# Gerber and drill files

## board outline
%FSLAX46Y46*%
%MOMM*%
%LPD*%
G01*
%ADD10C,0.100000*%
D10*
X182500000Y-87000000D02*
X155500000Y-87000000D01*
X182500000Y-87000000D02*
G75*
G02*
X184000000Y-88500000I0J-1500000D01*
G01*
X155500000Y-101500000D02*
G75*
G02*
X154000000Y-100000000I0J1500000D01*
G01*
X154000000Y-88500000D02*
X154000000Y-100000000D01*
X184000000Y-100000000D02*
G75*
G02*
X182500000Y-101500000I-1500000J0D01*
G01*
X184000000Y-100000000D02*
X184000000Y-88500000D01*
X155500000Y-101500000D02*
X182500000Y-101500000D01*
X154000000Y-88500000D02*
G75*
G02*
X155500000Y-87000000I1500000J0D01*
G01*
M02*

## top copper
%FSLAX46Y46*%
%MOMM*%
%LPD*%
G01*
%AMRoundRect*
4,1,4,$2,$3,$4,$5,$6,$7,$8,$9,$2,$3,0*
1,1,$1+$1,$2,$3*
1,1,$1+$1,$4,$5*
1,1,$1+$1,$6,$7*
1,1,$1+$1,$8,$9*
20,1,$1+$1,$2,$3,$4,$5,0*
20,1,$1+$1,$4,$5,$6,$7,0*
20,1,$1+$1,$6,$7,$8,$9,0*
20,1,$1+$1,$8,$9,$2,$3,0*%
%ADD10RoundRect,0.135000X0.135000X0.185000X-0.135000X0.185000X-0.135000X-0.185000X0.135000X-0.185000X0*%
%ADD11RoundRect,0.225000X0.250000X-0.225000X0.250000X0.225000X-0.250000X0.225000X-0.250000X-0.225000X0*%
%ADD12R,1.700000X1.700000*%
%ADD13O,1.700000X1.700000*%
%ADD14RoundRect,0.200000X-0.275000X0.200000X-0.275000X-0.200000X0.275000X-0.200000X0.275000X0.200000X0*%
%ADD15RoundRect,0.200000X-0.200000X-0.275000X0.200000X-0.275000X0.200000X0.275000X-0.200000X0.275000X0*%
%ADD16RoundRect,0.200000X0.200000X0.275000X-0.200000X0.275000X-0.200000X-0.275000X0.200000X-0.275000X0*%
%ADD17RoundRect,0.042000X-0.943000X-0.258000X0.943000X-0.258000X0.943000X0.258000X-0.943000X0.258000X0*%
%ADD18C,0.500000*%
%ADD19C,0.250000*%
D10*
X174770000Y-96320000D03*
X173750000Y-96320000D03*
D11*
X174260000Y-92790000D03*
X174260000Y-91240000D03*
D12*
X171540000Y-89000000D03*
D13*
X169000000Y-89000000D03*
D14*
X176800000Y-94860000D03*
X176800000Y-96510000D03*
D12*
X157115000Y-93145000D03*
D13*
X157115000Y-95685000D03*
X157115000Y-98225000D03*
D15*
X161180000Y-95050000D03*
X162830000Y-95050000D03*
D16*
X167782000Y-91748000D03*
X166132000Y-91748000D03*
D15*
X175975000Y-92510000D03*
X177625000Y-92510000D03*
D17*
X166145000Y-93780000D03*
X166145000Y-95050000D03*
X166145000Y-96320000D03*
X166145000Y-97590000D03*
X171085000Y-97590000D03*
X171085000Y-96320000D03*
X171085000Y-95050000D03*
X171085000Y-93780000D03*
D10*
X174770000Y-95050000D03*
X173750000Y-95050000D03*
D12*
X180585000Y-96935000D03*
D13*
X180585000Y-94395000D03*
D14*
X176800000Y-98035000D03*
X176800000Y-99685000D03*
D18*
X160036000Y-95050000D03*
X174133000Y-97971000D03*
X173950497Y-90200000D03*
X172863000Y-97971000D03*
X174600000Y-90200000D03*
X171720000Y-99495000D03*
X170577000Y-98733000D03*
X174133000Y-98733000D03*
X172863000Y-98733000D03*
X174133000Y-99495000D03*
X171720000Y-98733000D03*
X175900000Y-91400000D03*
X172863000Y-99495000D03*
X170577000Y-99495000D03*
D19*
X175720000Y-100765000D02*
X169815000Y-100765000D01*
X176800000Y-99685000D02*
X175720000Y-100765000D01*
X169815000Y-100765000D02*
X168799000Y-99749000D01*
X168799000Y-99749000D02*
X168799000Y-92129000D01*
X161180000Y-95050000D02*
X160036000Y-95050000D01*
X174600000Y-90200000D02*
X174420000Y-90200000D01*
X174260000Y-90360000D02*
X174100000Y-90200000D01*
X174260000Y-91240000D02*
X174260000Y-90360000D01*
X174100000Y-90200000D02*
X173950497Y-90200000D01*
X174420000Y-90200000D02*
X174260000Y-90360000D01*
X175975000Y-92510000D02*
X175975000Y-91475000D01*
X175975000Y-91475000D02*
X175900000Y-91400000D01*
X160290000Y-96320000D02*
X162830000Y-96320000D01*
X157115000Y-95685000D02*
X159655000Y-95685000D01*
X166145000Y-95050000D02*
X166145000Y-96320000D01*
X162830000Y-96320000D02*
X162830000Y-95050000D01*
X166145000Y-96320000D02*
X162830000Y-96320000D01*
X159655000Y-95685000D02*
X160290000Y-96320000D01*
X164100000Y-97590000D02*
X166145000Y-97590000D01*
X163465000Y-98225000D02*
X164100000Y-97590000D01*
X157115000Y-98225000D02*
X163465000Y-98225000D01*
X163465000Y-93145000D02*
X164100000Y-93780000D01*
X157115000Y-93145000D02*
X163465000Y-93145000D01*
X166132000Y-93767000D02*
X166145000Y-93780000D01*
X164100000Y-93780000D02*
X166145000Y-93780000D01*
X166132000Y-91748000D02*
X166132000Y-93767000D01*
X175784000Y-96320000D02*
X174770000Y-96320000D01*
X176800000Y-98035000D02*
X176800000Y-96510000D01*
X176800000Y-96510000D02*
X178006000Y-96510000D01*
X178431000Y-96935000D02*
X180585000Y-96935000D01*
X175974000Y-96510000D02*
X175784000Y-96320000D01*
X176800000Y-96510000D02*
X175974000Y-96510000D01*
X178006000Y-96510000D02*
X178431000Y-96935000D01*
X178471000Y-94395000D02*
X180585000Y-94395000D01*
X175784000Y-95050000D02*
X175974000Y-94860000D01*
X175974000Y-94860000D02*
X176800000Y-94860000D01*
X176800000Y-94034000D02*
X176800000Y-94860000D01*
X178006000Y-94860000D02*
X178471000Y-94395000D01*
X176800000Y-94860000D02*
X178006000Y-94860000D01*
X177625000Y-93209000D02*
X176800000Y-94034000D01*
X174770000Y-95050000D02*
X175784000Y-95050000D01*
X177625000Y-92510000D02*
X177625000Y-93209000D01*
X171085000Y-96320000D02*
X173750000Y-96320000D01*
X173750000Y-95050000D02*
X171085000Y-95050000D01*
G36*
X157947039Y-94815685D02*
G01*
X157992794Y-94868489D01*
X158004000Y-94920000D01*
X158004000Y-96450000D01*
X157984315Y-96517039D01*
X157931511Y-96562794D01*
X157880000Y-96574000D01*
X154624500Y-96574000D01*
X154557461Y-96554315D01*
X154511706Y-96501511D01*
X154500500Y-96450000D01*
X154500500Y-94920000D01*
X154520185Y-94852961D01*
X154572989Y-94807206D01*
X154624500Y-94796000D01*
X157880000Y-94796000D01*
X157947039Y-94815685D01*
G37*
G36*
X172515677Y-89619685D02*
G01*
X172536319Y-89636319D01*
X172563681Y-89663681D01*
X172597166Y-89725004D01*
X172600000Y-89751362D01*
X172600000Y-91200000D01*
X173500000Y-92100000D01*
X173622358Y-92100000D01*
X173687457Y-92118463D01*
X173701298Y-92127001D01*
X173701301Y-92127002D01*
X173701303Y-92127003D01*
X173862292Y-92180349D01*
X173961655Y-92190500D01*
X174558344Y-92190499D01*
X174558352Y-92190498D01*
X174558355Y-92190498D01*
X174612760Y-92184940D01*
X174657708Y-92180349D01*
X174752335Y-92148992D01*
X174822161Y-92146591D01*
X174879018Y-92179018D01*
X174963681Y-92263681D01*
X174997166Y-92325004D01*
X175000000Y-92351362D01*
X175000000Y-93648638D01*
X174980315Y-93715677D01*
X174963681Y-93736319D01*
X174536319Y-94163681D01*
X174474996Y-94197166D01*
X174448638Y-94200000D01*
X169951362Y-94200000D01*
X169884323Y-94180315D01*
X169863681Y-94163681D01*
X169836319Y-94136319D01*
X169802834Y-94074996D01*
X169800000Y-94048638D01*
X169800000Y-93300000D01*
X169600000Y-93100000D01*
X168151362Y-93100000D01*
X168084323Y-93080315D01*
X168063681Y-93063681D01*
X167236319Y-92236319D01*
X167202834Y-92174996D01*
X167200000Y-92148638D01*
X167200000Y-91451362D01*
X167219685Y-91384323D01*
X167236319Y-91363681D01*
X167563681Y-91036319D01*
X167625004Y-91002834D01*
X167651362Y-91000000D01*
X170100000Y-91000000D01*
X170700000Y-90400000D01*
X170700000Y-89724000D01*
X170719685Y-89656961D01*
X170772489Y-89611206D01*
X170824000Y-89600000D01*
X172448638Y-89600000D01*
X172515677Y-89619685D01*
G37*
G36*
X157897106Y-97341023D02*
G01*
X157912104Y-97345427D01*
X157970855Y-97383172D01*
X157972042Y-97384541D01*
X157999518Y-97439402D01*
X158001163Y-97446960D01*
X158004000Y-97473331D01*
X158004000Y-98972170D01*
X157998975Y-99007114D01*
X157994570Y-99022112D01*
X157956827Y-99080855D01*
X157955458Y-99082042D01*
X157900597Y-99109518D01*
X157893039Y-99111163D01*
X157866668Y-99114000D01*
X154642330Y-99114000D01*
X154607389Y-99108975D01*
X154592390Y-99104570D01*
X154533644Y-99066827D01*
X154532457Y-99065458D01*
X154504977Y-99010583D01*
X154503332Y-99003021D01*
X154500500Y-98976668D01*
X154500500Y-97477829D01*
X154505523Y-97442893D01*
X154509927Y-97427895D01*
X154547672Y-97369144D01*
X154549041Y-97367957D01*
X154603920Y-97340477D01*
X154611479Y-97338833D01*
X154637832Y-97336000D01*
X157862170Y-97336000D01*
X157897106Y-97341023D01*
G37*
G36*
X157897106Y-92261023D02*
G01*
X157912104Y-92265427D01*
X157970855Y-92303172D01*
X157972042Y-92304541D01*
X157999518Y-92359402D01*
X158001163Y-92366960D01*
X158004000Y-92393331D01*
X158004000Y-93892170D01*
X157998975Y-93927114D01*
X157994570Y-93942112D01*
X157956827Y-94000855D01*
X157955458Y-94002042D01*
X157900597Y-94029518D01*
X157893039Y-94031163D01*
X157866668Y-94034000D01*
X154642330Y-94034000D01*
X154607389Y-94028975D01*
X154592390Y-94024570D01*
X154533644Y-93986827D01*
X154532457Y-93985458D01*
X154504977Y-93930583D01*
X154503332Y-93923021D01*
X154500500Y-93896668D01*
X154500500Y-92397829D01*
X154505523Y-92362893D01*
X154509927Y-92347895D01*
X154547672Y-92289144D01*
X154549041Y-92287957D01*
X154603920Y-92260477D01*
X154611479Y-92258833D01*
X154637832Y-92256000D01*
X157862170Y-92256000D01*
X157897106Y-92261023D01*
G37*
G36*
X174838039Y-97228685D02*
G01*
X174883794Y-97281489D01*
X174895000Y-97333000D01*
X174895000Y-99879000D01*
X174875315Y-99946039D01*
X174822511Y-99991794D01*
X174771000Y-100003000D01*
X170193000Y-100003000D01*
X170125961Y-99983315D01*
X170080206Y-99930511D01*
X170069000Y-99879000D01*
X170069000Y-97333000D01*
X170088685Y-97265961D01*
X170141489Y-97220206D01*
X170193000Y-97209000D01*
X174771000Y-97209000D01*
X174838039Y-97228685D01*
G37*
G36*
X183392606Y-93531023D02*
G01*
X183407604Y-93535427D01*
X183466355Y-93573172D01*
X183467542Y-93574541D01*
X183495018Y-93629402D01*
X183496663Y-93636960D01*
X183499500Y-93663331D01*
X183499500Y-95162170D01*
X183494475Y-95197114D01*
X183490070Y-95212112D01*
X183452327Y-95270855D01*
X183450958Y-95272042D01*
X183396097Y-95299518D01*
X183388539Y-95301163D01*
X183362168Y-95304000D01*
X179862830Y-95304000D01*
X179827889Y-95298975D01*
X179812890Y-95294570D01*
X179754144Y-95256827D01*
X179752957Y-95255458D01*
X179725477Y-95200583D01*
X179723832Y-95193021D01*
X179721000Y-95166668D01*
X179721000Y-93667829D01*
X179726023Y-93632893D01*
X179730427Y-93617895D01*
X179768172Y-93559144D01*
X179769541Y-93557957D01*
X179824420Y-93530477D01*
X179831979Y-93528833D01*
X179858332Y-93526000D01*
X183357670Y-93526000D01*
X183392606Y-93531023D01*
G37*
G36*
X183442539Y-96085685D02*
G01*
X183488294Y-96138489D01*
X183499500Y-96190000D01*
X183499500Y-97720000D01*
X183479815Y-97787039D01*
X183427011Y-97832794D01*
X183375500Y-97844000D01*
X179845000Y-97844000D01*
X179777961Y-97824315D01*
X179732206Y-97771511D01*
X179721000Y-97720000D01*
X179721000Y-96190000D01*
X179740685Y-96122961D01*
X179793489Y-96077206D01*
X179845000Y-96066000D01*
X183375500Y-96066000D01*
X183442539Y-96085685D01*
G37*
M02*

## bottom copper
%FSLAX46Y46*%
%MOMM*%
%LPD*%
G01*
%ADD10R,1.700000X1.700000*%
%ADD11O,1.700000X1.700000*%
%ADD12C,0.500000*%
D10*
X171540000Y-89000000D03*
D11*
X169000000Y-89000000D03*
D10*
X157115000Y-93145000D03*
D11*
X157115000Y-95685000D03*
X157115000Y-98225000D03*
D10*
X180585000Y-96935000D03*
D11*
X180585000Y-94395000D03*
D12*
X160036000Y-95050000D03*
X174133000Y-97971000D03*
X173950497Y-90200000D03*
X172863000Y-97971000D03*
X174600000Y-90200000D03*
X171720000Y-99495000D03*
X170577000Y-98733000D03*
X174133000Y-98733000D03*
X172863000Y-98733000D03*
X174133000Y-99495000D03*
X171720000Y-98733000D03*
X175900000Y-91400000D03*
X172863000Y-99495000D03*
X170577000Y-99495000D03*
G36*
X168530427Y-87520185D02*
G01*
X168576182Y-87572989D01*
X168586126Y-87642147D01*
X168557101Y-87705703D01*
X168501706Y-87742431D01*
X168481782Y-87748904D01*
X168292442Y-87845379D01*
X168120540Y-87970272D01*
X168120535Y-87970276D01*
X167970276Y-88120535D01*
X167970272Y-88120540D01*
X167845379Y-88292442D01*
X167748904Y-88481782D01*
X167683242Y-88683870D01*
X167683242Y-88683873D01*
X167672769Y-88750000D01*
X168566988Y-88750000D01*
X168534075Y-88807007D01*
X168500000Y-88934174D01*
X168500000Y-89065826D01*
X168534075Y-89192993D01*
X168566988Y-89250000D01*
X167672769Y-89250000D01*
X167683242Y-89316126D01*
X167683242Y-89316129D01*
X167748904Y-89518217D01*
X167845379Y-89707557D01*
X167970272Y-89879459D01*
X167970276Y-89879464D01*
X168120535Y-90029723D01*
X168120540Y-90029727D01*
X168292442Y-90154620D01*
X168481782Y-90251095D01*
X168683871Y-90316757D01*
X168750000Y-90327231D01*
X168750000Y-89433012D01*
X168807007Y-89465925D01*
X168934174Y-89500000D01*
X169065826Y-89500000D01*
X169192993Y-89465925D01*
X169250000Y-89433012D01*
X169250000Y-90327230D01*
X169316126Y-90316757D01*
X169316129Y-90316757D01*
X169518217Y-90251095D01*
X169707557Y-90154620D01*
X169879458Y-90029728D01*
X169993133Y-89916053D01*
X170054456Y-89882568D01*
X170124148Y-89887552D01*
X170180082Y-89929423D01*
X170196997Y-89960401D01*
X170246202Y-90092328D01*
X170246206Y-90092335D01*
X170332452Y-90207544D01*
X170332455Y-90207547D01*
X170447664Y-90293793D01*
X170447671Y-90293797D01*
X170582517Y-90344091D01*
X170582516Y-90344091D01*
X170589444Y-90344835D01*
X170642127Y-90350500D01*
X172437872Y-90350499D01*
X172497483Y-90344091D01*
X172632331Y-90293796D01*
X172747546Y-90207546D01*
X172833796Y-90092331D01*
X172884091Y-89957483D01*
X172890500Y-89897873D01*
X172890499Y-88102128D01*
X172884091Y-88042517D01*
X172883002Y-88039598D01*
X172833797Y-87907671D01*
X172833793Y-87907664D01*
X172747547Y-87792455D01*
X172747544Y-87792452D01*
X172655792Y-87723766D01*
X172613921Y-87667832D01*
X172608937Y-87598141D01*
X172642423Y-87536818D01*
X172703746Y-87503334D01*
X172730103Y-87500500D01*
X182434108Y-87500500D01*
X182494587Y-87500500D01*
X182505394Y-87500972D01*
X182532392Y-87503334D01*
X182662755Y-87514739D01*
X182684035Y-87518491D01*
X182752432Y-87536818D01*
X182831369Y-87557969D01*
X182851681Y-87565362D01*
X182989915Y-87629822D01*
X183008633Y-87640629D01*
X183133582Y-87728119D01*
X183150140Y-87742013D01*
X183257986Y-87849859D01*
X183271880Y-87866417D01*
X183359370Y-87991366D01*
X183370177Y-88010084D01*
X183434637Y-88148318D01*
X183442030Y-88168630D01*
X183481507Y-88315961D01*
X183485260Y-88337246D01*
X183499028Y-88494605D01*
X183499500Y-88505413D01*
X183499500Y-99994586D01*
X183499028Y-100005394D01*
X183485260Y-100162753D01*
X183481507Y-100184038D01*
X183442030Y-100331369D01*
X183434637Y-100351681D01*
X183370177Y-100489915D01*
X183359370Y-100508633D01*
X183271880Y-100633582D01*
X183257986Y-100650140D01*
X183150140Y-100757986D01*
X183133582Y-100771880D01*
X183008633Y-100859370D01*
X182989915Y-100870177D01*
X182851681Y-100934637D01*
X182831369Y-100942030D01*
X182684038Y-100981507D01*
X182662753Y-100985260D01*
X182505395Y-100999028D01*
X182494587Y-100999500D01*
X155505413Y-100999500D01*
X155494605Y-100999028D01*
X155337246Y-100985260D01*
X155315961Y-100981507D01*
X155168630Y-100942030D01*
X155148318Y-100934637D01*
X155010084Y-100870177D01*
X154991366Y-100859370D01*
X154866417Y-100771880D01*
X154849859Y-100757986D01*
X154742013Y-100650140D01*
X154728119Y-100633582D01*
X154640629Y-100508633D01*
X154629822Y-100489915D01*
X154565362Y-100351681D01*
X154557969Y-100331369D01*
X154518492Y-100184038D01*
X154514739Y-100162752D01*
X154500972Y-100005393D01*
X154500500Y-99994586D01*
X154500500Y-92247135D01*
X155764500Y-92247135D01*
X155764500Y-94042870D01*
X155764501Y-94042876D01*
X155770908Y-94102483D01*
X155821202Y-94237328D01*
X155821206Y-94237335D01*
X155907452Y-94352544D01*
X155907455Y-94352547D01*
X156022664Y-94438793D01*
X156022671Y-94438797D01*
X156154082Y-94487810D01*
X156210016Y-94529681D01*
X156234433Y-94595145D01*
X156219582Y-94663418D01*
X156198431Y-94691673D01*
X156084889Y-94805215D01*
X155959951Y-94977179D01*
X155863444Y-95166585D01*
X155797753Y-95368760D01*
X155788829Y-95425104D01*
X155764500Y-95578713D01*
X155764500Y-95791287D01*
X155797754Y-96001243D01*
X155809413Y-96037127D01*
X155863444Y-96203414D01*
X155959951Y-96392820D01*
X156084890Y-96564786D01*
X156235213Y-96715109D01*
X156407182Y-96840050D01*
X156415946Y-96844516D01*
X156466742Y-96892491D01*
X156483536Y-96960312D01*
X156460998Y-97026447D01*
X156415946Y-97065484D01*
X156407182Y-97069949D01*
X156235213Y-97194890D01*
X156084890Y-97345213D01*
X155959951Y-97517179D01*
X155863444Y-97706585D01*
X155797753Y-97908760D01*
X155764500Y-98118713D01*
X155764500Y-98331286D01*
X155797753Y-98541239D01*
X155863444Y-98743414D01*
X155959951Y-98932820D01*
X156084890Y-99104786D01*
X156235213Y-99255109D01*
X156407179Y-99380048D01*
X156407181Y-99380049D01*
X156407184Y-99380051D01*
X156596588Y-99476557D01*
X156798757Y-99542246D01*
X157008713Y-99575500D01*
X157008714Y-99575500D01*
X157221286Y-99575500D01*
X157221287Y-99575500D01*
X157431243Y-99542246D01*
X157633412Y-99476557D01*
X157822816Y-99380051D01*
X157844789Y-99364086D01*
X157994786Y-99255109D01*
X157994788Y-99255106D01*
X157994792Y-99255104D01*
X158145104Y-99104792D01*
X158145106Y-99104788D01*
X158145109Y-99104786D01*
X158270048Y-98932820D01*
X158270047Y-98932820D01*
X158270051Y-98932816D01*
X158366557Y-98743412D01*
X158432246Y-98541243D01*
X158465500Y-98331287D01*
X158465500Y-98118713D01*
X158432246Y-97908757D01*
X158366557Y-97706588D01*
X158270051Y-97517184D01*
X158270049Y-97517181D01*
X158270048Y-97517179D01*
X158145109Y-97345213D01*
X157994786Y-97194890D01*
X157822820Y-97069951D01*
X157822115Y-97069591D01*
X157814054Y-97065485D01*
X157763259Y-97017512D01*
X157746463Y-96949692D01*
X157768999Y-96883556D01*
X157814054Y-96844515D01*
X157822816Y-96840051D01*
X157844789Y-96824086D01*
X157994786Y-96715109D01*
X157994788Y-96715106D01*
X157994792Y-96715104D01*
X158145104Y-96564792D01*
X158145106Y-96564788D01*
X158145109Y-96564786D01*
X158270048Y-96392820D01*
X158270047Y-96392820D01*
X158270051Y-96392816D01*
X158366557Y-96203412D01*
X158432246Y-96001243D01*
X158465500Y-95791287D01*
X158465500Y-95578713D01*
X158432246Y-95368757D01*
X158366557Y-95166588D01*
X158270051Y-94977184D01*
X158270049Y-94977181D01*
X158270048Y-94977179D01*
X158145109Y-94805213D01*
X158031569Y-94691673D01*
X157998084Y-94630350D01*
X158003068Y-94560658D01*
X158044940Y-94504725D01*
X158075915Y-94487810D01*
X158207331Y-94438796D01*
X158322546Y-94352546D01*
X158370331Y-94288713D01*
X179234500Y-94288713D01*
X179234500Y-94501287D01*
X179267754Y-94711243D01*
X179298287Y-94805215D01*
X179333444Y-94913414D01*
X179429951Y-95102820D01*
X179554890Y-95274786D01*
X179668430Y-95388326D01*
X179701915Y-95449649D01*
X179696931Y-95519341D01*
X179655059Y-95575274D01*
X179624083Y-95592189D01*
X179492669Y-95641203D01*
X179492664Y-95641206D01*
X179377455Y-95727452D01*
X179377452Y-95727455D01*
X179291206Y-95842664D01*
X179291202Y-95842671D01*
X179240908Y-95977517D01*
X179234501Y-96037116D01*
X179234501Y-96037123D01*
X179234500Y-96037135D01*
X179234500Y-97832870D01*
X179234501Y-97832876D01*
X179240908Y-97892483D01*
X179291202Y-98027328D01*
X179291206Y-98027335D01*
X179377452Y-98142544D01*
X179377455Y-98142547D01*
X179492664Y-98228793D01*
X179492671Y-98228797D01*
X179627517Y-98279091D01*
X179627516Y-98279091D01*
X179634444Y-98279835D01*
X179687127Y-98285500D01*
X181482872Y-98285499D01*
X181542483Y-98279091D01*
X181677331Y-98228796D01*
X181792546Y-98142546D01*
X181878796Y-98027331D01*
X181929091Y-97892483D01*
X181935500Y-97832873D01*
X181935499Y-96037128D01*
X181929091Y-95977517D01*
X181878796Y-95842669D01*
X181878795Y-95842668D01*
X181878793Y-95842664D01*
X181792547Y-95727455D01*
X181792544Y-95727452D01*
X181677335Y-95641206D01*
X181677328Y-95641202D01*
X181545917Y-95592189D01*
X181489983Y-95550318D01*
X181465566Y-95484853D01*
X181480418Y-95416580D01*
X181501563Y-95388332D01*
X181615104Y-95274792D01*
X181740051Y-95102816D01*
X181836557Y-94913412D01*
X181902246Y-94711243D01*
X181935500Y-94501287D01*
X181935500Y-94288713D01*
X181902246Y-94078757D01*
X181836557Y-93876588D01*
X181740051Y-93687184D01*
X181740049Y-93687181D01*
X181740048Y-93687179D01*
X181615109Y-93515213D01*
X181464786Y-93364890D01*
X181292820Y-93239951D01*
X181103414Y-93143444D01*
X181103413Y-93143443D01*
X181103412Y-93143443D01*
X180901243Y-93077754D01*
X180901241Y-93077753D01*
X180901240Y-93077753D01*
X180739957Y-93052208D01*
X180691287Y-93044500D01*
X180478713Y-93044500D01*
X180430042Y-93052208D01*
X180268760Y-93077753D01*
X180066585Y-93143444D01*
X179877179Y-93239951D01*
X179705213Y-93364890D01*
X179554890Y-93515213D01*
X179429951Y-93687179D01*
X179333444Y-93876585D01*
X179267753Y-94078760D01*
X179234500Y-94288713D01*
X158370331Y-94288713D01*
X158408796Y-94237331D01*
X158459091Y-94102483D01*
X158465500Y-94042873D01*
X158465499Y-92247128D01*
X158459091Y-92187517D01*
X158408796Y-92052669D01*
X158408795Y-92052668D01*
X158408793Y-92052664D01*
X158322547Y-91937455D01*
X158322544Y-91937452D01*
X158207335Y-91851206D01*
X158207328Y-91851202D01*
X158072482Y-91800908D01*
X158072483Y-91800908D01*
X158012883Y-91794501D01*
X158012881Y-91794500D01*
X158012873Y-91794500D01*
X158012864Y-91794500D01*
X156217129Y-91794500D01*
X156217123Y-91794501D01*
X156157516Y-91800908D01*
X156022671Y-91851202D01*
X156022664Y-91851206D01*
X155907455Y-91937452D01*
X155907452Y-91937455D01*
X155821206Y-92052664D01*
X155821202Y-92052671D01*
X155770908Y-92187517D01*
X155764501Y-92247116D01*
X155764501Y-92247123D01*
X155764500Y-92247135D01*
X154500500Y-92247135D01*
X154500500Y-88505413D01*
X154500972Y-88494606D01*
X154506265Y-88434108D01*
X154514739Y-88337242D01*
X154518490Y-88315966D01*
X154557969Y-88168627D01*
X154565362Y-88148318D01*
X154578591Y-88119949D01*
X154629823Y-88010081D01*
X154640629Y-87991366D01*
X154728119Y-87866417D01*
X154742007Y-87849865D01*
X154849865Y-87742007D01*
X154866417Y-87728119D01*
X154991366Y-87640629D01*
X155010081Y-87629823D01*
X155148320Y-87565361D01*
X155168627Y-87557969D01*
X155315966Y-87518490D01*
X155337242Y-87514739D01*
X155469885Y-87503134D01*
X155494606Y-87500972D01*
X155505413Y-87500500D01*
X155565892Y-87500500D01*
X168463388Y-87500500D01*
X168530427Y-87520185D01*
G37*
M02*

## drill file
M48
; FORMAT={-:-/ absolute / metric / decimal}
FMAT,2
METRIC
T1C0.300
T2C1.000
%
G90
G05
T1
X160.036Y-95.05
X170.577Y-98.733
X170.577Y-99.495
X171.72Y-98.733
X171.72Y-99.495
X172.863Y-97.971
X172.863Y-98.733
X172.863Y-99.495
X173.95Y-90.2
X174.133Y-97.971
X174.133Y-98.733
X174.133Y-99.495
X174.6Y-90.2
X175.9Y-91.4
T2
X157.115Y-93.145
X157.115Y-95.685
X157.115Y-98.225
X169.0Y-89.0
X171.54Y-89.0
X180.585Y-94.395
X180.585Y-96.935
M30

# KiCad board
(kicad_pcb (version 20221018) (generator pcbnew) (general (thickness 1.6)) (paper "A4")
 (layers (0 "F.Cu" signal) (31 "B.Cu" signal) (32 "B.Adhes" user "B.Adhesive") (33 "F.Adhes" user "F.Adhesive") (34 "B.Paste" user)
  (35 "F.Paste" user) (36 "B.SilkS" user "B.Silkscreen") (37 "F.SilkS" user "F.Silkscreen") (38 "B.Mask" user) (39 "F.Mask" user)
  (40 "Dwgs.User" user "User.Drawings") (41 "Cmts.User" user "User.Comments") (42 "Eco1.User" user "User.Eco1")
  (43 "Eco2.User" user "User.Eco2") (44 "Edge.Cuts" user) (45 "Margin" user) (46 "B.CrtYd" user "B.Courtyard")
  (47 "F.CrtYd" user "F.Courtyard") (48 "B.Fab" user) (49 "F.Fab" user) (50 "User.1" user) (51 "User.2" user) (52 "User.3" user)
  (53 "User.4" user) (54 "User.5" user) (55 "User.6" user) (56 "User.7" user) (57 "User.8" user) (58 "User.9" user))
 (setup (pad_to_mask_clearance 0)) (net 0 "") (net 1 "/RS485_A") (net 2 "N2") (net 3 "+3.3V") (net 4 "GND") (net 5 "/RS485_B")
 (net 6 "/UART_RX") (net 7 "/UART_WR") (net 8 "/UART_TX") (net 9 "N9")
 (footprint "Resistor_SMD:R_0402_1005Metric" (layer "F.Cu") (at 174.26 96.32 180)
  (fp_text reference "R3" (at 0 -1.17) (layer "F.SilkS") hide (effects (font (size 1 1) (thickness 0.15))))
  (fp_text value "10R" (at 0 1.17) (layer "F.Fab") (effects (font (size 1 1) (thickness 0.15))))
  (pad "1" smd roundrect (at -0.51 0 180) (size 0.54 0.64) (layers "F.Cu" "F.Paste" "F.Mask") (roundrect_rratio 0.25) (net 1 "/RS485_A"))
  (pad "2" smd roundrect (at 0.51 0 180) (size 0.54 0.64) (layers "F.Cu" "F.Paste" "F.Mask") (roundrect_rratio 0.25) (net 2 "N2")))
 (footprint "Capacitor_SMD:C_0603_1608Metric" (layer "F.Cu") (at 174.26 92.015 90)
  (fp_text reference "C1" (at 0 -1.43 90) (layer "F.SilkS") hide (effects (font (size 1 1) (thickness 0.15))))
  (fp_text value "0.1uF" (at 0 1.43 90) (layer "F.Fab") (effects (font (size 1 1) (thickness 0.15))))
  (pad "1" smd roundrect (at -0.775 0 90) (size 0.9 0.95) (layers "F.Cu" "F.Paste" "F.Mask") (roundrect_rratio 0.25) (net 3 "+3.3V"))
  (pad "2" smd roundrect (at 0.775 0 90) (size 0.9 0.95) (layers "F.Cu" "F.Paste" "F.Mask") (roundrect_rratio 0.25) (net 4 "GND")))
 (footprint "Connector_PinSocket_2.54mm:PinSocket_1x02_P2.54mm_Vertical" (layer "F.Cu") (at 171.54 89 -90)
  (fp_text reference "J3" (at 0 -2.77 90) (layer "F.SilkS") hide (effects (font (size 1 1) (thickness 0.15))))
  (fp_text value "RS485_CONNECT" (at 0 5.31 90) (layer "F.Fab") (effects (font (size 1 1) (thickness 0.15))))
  (pad "1" thru_hole rect (at 0 0 270) (size 1.7 1.7) (drill 1) (layers "*.Cu" "*.Mask") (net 3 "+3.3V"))
  (pad "2" thru_hole oval (at 0 2.54 270) (size 1.7 1.7) (drill 1) (layers "*.Cu" "*.Mask") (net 4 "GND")))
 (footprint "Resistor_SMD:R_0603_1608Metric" (layer "F.Cu") (at 176.8 95.685 -90)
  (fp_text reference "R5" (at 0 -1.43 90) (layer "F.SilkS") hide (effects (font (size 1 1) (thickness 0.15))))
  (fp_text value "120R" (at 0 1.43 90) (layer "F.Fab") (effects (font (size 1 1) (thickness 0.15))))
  (pad "1" smd roundrect (at -0.825 0 270) (size 0.8 0.95) (layers "F.Cu" "F.Paste" "F.Mask") (roundrect_rratio 0.25) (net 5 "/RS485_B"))
  (pad "2" smd roundrect (at 0.825 0 270) (size 0.8 0.95) (layers "F.Cu" "F.Paste" "F.Mask") (roundrect_rratio 0.25) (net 1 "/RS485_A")))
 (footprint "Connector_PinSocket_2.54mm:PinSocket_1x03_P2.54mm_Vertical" (layer "F.Cu") (at 157.115 93.145)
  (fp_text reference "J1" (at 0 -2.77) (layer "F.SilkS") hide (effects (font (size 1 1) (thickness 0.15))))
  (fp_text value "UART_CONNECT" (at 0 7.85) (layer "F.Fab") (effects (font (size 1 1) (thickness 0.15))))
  (pad "1" thru_hole rect (at 0 0) (size 1.7 1.7) (drill 1) (layers "*.Cu" "*.Mask") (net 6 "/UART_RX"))
  (pad "2" thru_hole oval (at 0 2.54) (size 1.7 1.7) (drill 1) (layers "*.Cu" "*.Mask") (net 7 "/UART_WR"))
  (pad "3" thru_hole oval (at 0 5.08) (size 1.7 1.7) (drill 1) (layers "*.Cu" "*.Mask") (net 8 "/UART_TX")))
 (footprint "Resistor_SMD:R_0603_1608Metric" (layer "F.Cu") (at 162.005 95.05)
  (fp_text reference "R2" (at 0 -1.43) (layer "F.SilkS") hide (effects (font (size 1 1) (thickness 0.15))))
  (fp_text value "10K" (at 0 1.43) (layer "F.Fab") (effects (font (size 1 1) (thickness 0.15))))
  (pad "1" smd roundrect (at -0.825 0) (size 0.8 0.95) (layers "F.Cu" "F.Paste" "F.Mask") (roundrect_rratio 0.25) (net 4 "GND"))
  (pad "2" smd roundrect (at 0.825 0) (size 0.8 0.95) (layers "F.Cu" "F.Paste" "F.Mask") (roundrect_rratio 0.25) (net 7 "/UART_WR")))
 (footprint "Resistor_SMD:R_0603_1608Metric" (layer "F.Cu") (at 166.957 91.748 180)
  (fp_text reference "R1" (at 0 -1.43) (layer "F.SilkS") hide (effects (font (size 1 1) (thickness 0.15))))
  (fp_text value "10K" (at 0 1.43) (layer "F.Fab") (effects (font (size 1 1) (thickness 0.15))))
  (pad "1" smd roundrect (at -0.825 0 180) (size 0.8 0.95) (layers "F.Cu" "F.Paste" "F.Mask") (roundrect_rratio 0.25) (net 3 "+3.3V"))
  (pad "2" smd roundrect (at 0.825 0 180) (size 0.8 0.95) (layers "F.Cu" "F.Paste" "F.Mask") (roundrect_rratio 0.25) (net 6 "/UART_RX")))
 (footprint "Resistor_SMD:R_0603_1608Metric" (layer "F.Cu") (at 176.8 92.51)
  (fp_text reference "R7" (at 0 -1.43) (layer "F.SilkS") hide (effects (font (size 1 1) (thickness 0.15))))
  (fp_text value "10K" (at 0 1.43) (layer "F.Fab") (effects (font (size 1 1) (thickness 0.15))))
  (pad "1" smd roundrect (at -0.825 0) (size 0.8 0.95) (layers "F.Cu" "F.Paste" "F.Mask") (roundrect_rratio 0.25) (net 4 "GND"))
  (pad "2" smd roundrect (at 0.825 0) (size 0.8 0.95) (layers "F.Cu" "F.Paste" "F.Mask") (roundrect_rratio 0.25) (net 5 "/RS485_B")))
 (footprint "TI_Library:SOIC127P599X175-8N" (layer "F.Cu") (at 168.615 95.685)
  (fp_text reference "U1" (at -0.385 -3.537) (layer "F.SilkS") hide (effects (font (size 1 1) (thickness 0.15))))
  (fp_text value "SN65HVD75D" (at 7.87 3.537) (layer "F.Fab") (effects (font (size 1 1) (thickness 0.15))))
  (pad "1" smd roundrect (at -2.47 -1.905) (size 1.97 0.6) (layers "F.Cu" "F.Paste" "F.Mask") (roundrect_rratio 0.07) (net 6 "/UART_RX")
   (solder_mask_margin 0.102))
  (pad "2" smd roundrect (at -2.47 -0.635) (size 1.97 0.6) (layers "F.Cu" "F.Paste" "F.Mask") (roundrect_rratio 0.07) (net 7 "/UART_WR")
   (solder_mask_margin 0.102))
  (pad "3" smd roundrect (at -2.47 0.635) (size 1.97 0.6) (layers "F.Cu" "F.Paste" "F.Mask") (roundrect_rratio 0.07) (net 7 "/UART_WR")
   (solder_mask_margin 0.102))
  (pad "4" smd roundrect (at -2.47 1.905) (size 1.97 0.6) (layers "F.Cu" "F.Paste" "F.Mask") (roundrect_rratio 0.07) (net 8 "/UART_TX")
   (solder_mask_margin 0.102))
  (pad "5" smd roundrect (at 2.47 1.905) (size 1.97 0.6) (layers "F.Cu" "F.Paste" "F.Mask") (roundrect_rratio 0.07) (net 4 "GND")
   (solder_mask_margin 0.102))
  (pad "6" smd roundrect (at 2.47 0.635) (size 1.97 0.6) (layers "F.Cu" "F.Paste" "F.Mask") (roundrect_rratio 0.07) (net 2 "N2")
   (solder_mask_margin 0.102))
  (pad "7" smd roundrect (at 2.47 -0.635) (size 1.97 0.6) (layers "F.Cu" "F.Paste" "F.Mask") (roundrect_rratio 0.07) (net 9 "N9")
   (solder_mask_margin 0.102))
  (pad "8" smd roundrect (at 2.47 -1.905) (size 1.97 0.6) (layers "F.Cu" "F.Paste" "F.Mask") (roundrect_rratio 0.07) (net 3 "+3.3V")
   (solder_mask_margin 0.102)))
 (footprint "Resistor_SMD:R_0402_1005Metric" (layer "F.Cu") (at 174.26 95.05 180)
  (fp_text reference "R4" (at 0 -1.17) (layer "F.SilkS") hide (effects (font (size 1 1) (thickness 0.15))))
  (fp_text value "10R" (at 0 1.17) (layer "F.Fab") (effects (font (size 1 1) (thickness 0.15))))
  (pad "1" smd roundrect (at -0.51 0 180) (size 0.54 0.64) (layers "F.Cu" "F.Paste" "F.Mask") (roundrect_rratio 0.25) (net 5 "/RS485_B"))
  (pad "2" smd roundrect (at 0.51 0 180) (size 0.54 0.64) (layers "F.Cu" "F.Paste" "F.Mask") (roundrect_rratio 0.25) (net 9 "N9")))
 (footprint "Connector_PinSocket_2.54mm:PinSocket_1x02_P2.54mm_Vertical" (layer "F.Cu") (at 180.585 96.935 180)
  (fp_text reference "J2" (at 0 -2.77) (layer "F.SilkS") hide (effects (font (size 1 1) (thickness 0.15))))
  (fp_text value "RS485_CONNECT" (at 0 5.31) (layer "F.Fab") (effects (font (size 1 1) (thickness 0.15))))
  (pad "1" thru_hole rect (at 0 0 180) (size 1.7 1.7) (drill 1) (layers "*.Cu" "*.Mask") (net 1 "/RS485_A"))
  (pad "2" thru_hole oval (at 0 2.54 180) (size 1.7 1.7) (drill 1) (layers "*.Cu" "*.Mask") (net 5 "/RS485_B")))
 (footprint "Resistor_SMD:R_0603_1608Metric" (layer "F.Cu") (at 176.8 98.86 -90)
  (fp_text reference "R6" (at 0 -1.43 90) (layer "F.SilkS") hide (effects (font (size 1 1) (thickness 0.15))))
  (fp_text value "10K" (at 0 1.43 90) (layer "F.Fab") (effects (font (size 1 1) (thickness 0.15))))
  (pad "1" smd roundrect (at -0.825 0 270) (size 0.8 0.95) (layers "F.Cu" "F.Paste" "F.Mask") (roundrect_rratio 0.25) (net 1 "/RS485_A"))
  (pad "2" smd roundrect (at 0.825 0 270) (size 0.8 0.95) (layers "F.Cu" "F.Paste" "F.Mask") (roundrect_rratio 0.25) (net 3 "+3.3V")))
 (gr_line (start 182.5 87) (end 155.5 87) (stroke (width 0.1) (type default)) (layer "Edge.Cuts"))
 (gr_arc (start 182.5 87) (mid 183.56066 87.43934) (end 184 88.5) (stroke (width 0.1) (type default)) (layer "Edge.Cuts"))
 (gr_arc (start 155.5 101.5) (mid 154.43934 101.06066) (end 154 100) (stroke (width 0.1) (type default)) (layer "Edge.Cuts"))
 (gr_line (start 154 88.5) (end 154 100) (stroke (width 0.1) (type default)) (layer "Edge.Cuts"))
 (gr_arc (start 184 100) (mid 183.56066 101.06066) (end 182.5 101.5) (stroke (width 0.1) (type default)) (layer "Edge.Cuts"))
 (gr_line (start 184 100) (end 184 88.5) (stroke (width 0.1) (type default)) (layer "Edge.Cuts"))
 (gr_line (start 155.5 101.5) (end 182.5 101.5) (stroke (width 0.1) (type default)) (layer "Edge.Cuts"))
 (gr_arc (start 154 88.5) (mid 154.43934 87.43934) (end 155.5 87) (stroke (width 0.1) (type default)) (layer "Edge.Cuts"))
 (segment (start 175.72 100.765) (end 169.815 100.765) (width 0.25) (layer "F.Cu") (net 3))
 (segment (start 176.8 99.685) (end 175.72 100.765) (width 0.25) (layer "F.Cu") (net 3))
 (segment (start 169.815 100.765) (end 168.799 99.749) (width 0.25) (layer "F.Cu") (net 3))
 (segment (start 168.799 99.749) (end 168.799 92.129) (width 0.25) (layer "F.Cu") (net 3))
 (segment (start 161.18 95.05) (end 160.036 95.05) (width 0.25) (layer "F.Cu") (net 4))
 (segment (start 174.6 90.2) (end 174.42 90.2) (width 0.25) (layer "F.Cu") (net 4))
 (segment (start 174.26 90.36) (end 174.1 90.2) (width 0.25) (layer "F.Cu") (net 4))
 (segment (start 174.26 91.24) (end 174.26 90.36) (width 0.25) (layer "F.Cu") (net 4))
 (segment (start 174.1 90.2) (end 173.950497 90.2) (width 0.25) (layer "F.Cu") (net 4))
 (segment (start 174.42 90.2) (end 174.26 90.36) (width 0.25) (layer "F.Cu") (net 4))
 (segment (start 175.975 92.51) (end 175.975 91.475) (width 0.25) (layer "F.Cu") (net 4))
 (segment (start 175.975 91.475) (end 175.9 91.4) (width 0.25) (layer "F.Cu") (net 4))
 (via (at 160.036 95.05) (size 0.5) (drill 0.3) (layers "F.Cu" "B.Cu") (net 4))
 (via (at 174.133 97.971) (size 0.5) (drill 0.3) (layers "F.Cu" "B.Cu") (free) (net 4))
 (via (at 173.950497 90.2) (size 0.5) (drill 0.3) (layers "F.Cu" "B.Cu") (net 4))
 (via (at 172.863 97.971) (size 0.5) (drill 0.3) (layers "F.Cu" "B.Cu") (free) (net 4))
 (via (at 174.6 90.2) (size 0.5) (drill 0.3) (layers "F.Cu" "B.Cu") (free) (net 4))
 (via (at 171.72 99.495) (size 0.5) (drill 0.3) (layers "F.Cu" "B.Cu") (free) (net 4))
 (via (at 170.577 98.733) (size 0.5) (drill 0.3) (layers "F.Cu" "B.Cu") (free) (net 4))
 (via (at 174.133 98.733) (size 0.5) (drill 0.3) (layers "F.Cu" "B.Cu") (free) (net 4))
 (via (at 172.863 98.733) (size 0.5) (drill 0.3) (layers "F.Cu" "B.Cu") (free) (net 4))
 (via (at 174.133 99.495) (size 0.5) (drill 0.3) (layers "F.Cu" "B.Cu") (free) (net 4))
 (via (at 171.72 98.733) (size 0.5) (drill 0.3) (layers "F.Cu" "B.Cu") (free) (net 4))
 (via (at 175.9 91.4) (size 0.5) (drill 0.3) (layers "F.Cu" "B.Cu") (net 4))
 (via (at 172.863 99.495) (size 0.5) (drill 0.3) (layers "F.Cu" "B.Cu") (free) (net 4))
 (via (at 170.577 99.495) (size 0.5) (drill 0.3) (layers "F.Cu" "B.Cu") (free) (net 4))
 (segment (start 160.29 96.32) (end 162.83 96.32) (width 0.25) (layer "F.Cu") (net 7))
 (segment (start 157.115 95.685) (end 159.655 95.685) (width 0.25) (layer "F.Cu") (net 7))
 (segment (start 166.145 95.05) (end 166.145 96.32) (width 0.25) (layer "F.Cu") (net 7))
 (segment (start 162.83 96.32) (end 162.83 95.05) (width 0.25) (layer "F.Cu") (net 7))
 (segment (start 166.145 96.32) (end 162.83 96.32) (width 0.25) (layer "F.Cu") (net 7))
 (segment (start 159.655 95.685) (end 160.29 96.32) (width 0.25) (layer "F.Cu") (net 7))
 (segment (start 164.1 97.59) (end 166.145 97.59) (width 0.25) (layer "F.Cu") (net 8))
 (segment (start 163.465 98.225) (end 164.1 97.59) (width 0.25) (layer "F.Cu") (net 8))
 (segment (start 157.115 98.225) (end 163.465 98.225) (width 0.25) (layer "F.Cu") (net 8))
 (segment (start 163.465 93.145) (end 164.1 93.78) (width 0.25) (layer "F.Cu") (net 6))
 (segment (start 157.115 93.145) (end 163.465 93.145) (width 0.25) (layer "F.Cu") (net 6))
 (segment (start 166.132 93.767) (end 166.145 93.78) (width 0.25) (layer "F.Cu") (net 6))
 (segment (start 164.1 93.78) (end 166.145 93.78) (width 0.25) (layer "F.Cu") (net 6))
 (segment (start 166.132 91.748) (end 166.132 93.767) (width 0.25) (layer "F.Cu") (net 6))
 (segment (start 175.784 96.32) (end 174.77 96.32) (width 0.25) (layer "F.Cu") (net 1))
 (segment (start 176.8 98.035) (end 176.8 96.51) (width 0.25) (layer "F.Cu") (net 1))
 (segment (start 176.8 96.51) (end 178.006 96.51) (width 0.25) (layer "F.Cu") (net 1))
 (segment (start 178.431 96.935) (end 180.585 96.935) (width 0.25) (layer "F.Cu") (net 1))
 (segment (start 175.974 96.51) (end 175.784 96.32) (width 0.25) (layer "F.Cu") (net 1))
 (segment (start 176.8 96.51) (end 175.974 96.51) (width 0.25) (layer "F.Cu") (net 1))
 (segment (start 178.006 96.51) (end 178.431 96.935) (width 0.25) (layer "F.Cu") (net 1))
 (segment (start 178.471 94.395) (end 180.585 94.395) (width 0.25) (layer "F.Cu") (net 5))
 (segment (start 175.784 95.05) (end 175.974 94.86) (width 0.25) (layer "F.Cu") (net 5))
 (segment (start 175.974 94.86) (end 176.8 94.86) (width 0.25) (layer "F.Cu") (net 5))
 (segment (start 176.8 94.034) (end 176.8 94.86) (width 0.25) (layer "F.Cu") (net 5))
 (segment (start 178.006 94.86) (end 178.471 94.395) (width 0.25) (layer "F.Cu") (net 5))
 (segment (start 176.8 94.86) (end 178.006 94.86) (width 0.25) (layer "F.Cu") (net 5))
 (segment (start 177.625 93.209) (end 176.8 94.034) (width 0.25) (layer "F.Cu") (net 5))
 (segment (start 174.77 95.05) (end 175.784 95.05) (width 0.25) (layer "F.Cu") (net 5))
 (segment (start 177.625 92.51) (end 177.625 93.209) (width 0.25) (layer "F.Cu") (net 5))
 (segment (start 171.085 96.32) (end 173.75 96.32) (width 0.25) (layer "F.Cu") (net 2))
 (segment (start 173.75 95.05) (end 171.085 95.05) (width 0.25) (layer "F.Cu") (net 9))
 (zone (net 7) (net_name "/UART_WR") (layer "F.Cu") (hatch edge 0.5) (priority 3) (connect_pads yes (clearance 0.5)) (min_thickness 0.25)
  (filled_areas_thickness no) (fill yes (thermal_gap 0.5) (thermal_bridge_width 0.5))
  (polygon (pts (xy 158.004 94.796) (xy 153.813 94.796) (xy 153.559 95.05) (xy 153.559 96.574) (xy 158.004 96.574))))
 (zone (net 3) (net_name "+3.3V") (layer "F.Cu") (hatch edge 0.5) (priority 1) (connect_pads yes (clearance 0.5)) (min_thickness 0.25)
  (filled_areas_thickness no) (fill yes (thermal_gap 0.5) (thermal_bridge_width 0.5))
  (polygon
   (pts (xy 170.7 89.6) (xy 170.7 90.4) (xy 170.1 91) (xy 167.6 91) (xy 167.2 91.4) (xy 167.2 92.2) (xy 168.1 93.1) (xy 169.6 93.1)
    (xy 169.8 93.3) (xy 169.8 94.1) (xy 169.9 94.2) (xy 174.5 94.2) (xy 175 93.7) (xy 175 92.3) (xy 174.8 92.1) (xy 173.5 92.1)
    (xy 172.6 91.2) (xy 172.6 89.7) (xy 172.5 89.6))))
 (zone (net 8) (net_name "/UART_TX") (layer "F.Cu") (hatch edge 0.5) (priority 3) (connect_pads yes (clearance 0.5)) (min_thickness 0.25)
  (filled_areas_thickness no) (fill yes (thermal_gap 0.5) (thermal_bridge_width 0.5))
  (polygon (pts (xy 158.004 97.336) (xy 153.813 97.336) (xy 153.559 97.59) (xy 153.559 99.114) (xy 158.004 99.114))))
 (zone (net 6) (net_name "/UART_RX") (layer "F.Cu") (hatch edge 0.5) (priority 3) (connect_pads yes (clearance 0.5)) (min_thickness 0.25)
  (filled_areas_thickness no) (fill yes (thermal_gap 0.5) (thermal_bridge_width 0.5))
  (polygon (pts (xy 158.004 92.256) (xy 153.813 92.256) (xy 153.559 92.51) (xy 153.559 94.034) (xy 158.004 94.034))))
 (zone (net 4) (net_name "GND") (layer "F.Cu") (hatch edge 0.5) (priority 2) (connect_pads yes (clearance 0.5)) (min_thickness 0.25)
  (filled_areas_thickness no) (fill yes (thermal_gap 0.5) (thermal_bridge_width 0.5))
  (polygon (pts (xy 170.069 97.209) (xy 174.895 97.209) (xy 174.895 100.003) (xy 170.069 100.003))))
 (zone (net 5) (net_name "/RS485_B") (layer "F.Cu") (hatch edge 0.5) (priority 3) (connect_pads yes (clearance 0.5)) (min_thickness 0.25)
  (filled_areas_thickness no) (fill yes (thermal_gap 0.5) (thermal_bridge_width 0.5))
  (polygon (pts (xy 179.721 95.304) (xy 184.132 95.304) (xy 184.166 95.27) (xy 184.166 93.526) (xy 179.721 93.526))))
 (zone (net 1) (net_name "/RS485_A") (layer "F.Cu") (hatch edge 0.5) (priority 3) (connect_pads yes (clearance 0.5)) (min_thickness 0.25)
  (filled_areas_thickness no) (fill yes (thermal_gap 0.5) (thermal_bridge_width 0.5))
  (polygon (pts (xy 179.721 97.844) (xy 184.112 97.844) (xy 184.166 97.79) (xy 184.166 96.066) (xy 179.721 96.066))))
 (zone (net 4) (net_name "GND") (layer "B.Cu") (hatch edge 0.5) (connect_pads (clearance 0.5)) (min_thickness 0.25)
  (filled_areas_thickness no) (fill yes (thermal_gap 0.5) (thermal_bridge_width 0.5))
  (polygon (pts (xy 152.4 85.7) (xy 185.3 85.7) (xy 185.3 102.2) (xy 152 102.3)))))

